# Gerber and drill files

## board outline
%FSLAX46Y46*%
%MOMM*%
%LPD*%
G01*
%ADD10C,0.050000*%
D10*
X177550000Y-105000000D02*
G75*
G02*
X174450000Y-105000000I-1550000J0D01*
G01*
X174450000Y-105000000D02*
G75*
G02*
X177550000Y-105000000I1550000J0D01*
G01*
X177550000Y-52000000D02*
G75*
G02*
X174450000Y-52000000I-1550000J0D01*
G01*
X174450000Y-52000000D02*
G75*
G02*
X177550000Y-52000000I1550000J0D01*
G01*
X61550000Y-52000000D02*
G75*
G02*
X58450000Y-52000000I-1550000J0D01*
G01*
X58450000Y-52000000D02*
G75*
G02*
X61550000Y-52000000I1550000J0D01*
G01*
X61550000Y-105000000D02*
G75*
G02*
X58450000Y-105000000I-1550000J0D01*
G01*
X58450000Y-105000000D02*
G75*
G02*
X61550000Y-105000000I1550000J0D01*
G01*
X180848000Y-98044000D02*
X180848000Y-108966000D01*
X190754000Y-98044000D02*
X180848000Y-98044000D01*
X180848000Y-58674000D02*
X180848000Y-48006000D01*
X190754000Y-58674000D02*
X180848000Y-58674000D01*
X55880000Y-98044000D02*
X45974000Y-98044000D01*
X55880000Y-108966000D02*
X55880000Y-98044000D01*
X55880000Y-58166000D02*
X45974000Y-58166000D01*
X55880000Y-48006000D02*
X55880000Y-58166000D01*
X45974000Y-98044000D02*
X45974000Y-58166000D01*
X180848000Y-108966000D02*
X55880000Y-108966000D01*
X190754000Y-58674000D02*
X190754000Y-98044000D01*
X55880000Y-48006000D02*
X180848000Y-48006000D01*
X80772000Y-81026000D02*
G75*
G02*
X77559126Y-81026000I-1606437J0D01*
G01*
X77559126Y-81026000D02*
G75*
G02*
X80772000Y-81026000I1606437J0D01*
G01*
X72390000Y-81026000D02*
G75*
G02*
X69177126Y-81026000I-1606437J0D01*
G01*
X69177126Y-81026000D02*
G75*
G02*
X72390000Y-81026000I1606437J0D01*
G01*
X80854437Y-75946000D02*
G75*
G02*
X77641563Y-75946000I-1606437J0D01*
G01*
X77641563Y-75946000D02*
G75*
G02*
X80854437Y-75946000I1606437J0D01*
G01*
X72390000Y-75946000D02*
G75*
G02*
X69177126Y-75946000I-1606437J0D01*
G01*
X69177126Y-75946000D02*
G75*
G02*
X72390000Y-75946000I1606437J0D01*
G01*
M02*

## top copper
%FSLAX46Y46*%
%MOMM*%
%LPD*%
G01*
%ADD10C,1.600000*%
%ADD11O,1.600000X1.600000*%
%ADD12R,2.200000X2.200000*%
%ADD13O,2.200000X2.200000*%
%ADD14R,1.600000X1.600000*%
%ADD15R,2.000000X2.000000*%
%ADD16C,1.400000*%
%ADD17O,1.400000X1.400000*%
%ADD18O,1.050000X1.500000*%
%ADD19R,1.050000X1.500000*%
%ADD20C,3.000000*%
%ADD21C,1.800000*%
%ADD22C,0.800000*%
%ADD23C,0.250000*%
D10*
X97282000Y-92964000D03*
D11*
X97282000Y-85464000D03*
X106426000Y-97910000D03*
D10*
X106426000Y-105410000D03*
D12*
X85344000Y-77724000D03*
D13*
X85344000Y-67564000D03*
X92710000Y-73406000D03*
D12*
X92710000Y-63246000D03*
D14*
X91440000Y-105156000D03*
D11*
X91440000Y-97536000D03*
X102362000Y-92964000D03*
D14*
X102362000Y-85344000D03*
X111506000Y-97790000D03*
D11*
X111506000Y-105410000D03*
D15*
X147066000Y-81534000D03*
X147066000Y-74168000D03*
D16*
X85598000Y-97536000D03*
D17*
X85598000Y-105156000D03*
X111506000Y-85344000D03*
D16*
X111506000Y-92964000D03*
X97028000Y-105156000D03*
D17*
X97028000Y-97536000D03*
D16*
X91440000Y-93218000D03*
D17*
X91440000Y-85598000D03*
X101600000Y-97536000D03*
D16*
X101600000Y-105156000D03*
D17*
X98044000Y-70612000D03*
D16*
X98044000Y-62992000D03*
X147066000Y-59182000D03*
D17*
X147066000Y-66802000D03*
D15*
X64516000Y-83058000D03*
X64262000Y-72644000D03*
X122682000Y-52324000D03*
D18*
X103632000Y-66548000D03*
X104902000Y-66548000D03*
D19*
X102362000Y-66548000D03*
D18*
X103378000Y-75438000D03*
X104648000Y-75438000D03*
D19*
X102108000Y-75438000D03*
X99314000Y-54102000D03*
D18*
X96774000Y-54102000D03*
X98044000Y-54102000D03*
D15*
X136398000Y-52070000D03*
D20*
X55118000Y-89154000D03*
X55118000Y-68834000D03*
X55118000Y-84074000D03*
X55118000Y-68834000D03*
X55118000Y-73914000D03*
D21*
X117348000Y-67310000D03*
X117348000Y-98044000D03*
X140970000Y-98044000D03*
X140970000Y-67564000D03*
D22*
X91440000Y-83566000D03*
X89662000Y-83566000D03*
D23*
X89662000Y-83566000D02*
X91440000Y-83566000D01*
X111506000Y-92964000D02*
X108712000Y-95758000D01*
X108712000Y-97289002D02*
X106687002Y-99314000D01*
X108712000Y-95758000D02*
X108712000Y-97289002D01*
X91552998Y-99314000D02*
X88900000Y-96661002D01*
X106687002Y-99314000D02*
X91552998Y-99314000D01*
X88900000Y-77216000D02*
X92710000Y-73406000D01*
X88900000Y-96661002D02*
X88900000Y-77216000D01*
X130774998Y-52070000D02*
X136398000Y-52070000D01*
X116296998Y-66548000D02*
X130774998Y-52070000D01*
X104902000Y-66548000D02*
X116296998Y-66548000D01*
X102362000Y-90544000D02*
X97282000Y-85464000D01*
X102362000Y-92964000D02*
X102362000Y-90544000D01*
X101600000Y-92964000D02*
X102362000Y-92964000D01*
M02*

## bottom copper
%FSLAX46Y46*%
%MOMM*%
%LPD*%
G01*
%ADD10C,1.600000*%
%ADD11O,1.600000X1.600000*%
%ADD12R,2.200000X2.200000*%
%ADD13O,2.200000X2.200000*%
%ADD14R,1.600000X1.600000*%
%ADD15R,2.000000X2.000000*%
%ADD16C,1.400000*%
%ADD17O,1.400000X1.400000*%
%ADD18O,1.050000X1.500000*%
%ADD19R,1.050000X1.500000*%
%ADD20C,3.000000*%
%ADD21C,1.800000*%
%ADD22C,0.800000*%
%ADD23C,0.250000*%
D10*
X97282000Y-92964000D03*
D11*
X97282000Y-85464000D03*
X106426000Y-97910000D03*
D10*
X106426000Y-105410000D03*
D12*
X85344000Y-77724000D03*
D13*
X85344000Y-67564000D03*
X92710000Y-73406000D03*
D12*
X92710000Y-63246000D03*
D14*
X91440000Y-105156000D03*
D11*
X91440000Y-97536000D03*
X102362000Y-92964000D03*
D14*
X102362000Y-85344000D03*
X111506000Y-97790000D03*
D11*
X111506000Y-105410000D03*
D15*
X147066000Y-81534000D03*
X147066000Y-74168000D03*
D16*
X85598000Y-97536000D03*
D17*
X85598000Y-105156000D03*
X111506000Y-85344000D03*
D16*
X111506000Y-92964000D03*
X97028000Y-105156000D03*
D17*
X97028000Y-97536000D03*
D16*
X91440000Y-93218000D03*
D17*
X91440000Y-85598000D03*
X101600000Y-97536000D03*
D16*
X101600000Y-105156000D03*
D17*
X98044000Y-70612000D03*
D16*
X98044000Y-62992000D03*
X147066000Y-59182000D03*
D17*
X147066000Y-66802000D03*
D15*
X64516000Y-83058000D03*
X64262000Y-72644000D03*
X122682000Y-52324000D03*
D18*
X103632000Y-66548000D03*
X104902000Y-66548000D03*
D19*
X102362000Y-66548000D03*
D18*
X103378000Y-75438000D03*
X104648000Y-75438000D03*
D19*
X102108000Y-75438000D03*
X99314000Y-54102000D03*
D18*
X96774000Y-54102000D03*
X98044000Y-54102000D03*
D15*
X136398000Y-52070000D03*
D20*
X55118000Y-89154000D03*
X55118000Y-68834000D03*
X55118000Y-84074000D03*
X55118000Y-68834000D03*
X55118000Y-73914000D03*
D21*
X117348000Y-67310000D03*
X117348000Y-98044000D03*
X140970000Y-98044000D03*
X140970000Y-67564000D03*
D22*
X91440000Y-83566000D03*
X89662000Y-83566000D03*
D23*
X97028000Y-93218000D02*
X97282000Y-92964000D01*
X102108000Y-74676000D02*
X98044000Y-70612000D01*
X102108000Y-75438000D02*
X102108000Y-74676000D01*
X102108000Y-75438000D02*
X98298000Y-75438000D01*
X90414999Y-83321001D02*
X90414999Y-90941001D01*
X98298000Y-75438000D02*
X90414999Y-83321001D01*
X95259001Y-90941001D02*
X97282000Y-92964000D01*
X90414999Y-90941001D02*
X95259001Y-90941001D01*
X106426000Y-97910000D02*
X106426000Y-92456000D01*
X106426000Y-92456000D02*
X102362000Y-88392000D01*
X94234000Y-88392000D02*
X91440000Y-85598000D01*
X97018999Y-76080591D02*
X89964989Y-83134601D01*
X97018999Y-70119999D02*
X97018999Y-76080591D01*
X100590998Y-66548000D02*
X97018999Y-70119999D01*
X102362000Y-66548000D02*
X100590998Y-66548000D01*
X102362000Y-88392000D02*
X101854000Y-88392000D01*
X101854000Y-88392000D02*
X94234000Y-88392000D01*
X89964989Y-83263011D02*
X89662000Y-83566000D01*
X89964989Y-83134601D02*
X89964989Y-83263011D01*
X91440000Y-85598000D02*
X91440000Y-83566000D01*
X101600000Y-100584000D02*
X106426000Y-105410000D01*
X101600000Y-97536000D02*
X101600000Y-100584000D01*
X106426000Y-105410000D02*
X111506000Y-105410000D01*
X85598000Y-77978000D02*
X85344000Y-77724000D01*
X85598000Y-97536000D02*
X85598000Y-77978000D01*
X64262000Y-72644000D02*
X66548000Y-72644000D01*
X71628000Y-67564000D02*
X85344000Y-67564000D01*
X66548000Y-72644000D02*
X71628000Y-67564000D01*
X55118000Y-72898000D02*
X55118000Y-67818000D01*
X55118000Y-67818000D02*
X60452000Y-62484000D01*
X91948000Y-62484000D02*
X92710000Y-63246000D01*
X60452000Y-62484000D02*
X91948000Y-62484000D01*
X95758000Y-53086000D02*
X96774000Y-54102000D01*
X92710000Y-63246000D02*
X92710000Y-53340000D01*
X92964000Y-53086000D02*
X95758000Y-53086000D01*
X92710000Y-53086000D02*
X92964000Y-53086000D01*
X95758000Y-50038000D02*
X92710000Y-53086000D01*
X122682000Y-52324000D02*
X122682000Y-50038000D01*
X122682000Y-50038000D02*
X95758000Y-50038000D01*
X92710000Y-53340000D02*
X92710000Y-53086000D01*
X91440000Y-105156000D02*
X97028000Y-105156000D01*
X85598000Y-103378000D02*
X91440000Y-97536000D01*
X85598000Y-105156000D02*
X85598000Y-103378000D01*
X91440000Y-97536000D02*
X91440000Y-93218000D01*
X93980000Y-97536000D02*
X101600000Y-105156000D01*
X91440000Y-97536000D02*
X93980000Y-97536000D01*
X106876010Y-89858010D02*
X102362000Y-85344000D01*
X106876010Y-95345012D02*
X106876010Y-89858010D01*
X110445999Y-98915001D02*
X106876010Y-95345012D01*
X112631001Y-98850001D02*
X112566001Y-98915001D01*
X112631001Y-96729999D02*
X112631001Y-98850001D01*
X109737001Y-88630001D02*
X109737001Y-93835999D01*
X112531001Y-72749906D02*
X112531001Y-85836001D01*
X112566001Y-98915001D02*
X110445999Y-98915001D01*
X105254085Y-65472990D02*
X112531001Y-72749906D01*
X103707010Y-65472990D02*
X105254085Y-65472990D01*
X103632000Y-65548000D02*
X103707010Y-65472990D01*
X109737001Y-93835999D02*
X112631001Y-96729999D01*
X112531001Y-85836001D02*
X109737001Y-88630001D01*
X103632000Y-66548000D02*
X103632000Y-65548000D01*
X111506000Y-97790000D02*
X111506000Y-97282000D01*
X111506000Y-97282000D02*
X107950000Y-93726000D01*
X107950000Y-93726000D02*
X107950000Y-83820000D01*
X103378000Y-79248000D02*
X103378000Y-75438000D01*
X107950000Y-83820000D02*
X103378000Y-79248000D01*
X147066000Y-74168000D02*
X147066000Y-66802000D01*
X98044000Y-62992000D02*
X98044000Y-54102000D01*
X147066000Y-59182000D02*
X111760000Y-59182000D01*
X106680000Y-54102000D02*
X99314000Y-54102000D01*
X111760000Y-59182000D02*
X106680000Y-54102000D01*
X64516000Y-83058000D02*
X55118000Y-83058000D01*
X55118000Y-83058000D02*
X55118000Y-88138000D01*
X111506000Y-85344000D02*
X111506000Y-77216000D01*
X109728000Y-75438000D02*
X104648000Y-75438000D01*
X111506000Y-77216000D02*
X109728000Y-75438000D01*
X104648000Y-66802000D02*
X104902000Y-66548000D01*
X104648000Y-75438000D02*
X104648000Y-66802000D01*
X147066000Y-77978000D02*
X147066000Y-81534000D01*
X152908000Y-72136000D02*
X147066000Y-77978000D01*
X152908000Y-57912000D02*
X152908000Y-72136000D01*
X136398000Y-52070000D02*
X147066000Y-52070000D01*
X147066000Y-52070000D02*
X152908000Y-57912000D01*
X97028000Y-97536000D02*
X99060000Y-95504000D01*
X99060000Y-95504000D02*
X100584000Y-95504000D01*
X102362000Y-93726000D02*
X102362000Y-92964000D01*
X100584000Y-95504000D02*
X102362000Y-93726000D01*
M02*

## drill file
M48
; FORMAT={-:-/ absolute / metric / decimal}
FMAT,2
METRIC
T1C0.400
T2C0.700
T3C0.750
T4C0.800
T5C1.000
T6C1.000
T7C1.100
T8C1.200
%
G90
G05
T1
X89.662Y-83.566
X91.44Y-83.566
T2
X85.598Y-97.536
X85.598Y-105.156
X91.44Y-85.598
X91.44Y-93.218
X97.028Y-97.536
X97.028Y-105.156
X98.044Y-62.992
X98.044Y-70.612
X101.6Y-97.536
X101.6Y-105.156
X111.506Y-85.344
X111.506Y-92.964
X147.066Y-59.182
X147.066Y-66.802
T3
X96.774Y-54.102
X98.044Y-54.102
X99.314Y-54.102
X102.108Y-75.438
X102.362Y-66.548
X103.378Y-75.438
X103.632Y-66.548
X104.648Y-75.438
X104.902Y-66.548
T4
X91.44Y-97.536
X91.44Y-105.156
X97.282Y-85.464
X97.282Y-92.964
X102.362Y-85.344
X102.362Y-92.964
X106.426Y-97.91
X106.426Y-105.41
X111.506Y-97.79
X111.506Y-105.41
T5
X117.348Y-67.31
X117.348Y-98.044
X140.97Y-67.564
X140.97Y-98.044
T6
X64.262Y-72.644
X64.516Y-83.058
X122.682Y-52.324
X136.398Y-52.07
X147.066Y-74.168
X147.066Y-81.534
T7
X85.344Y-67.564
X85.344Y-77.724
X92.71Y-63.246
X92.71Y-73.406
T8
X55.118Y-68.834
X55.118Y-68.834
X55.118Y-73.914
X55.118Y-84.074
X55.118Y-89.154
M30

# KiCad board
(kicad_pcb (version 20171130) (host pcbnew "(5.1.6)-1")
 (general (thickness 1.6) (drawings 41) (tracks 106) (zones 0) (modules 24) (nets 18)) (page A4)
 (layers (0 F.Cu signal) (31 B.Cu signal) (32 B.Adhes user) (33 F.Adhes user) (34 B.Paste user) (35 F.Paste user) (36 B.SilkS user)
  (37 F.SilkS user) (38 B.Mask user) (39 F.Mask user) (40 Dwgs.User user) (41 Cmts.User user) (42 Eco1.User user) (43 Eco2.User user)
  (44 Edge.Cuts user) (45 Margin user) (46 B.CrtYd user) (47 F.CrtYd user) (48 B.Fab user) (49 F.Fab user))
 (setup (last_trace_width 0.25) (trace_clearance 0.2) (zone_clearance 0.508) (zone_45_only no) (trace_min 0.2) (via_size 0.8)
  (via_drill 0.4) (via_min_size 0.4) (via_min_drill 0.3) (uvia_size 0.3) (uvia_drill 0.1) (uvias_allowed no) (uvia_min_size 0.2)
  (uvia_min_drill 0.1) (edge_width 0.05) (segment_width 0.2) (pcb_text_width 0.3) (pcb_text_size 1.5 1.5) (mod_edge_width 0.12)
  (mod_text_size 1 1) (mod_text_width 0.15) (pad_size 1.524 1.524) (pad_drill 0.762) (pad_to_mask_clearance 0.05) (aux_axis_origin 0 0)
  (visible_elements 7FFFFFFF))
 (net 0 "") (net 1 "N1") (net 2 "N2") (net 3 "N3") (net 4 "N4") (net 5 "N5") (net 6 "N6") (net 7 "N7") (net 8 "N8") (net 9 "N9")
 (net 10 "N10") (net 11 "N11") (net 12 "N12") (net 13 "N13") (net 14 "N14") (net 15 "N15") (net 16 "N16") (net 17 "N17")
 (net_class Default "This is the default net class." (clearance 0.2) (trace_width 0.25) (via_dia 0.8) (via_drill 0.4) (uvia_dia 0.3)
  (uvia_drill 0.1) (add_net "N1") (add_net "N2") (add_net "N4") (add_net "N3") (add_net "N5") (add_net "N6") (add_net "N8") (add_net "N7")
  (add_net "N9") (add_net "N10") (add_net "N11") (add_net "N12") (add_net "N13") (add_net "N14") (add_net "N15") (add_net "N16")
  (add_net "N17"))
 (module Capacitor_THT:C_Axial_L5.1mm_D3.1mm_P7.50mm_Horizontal (layer F.Cu) (at 97.282 92.964 90)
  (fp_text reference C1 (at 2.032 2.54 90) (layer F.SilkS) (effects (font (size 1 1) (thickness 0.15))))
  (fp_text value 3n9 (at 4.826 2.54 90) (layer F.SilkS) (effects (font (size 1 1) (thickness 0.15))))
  (pad 1 thru_hole circle (at 0 0 90) (size 1.6 1.6) (drill 0.8) (layers *.Cu *.Mask) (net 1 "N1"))
  (pad 2 thru_hole oval (at 7.5 0 90) (size 1.6 1.6) (drill 0.8) (layers *.Cu *.Mask) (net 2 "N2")))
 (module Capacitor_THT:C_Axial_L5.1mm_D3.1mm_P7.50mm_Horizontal (layer F.Cu) (at 106.426 105.41 90)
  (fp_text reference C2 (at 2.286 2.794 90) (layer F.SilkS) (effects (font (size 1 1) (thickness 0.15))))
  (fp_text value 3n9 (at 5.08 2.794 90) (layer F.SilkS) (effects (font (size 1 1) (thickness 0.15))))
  (pad 2 thru_hole oval (at 7.5 0 90) (size 1.6 1.6) (drill 0.8) (layers *.Cu *.Mask) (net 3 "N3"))
  (pad 1 thru_hole circle (at 0 0 90) (size 1.6 1.6) (drill 0.8) (layers *.Cu *.Mask) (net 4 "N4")))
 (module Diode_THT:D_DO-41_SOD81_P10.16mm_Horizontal (layer F.Cu) (at 85.344 77.724 90)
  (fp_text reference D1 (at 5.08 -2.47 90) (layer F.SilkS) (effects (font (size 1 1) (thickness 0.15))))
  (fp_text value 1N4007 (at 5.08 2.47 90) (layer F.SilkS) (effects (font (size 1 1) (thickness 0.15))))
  (pad 1 thru_hole rect (at 0 0 90) (size 2.2 2.2) (drill 1.1) (layers *.Cu *.Mask) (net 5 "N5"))
  (pad 2 thru_hole oval (at 10.16 0 90) (size 2.2 2.2) (drill 1.1) (layers *.Cu *.Mask) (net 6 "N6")))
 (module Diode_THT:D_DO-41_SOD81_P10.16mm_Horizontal (layer F.Cu) (at 92.71 63.246 270)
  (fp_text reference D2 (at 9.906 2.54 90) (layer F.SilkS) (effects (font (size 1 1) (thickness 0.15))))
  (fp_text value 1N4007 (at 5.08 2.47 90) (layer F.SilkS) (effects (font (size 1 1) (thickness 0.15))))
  (pad 2 thru_hole oval (at 10.16 0 270) (size 2.2 2.2) (drill 1.1) (layers *.Cu *.Mask) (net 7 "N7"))
  (pad 1 thru_hole rect (at 0 0 270) (size 2.2 2.2) (drill 1.1) (layers *.Cu *.Mask) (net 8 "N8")))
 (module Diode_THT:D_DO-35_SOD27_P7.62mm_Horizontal (layer F.Cu) (at 91.44 105.156 90)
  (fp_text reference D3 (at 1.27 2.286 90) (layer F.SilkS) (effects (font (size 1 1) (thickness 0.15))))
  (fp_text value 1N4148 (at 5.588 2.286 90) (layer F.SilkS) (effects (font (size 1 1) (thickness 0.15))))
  (pad 1 thru_hole rect (at 0 0 90) (size 1.6 1.6) (drill 0.8) (layers *.Cu *.Mask) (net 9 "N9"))
  (pad 2 thru_hole oval (at 7.62 0 90) (size 1.6 1.6) (drill 0.8) (layers *.Cu *.Mask) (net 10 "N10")))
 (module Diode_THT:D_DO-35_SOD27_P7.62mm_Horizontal (layer F.Cu) (at 102.362 85.344 270)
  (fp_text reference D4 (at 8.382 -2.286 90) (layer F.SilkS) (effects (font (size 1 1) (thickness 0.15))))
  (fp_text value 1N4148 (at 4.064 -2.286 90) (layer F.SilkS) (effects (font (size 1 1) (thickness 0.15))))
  (pad 2 thru_hole oval (at 7.62 0 270) (size 1.6 1.6) (drill 0.8) (layers *.Cu *.Mask) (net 2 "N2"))
  (pad 1 thru_hole rect (at 0 0 270) (size 1.6 1.6) (drill 0.8) (layers *.Cu *.Mask) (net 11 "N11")))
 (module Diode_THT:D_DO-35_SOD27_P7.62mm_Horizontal (layer F.Cu) (at 111.506 97.79 270)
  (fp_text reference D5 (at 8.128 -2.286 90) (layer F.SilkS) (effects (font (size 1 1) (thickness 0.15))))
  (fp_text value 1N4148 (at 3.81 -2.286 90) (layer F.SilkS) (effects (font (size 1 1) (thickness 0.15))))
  (pad 1 thru_hole rect (at 0 0 270) (size 1.6 1.6) (drill 0.8) (layers *.Cu *.Mask) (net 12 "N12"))
  (pad 2 thru_hole oval (at 7.62 0 270) (size 1.6 1.6) (drill 0.8) (layers *.Cu *.Mask) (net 4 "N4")))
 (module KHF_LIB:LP (layer F.Cu) (at 147.066 81.534)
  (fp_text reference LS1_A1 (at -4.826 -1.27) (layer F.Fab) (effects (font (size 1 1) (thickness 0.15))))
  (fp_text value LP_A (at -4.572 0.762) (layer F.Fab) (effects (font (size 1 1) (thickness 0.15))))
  (pad 1 thru_hole rect (at 0 0) (size 2 2) (drill 1) (layers *.Cu *.Mask) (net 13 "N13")))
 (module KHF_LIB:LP (layer F.Cu) (at 147.066 74.168)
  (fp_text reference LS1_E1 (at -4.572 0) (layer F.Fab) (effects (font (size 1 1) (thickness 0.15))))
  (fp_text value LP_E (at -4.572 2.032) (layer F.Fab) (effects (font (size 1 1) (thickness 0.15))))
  (pad 1 thru_hole rect (at 0 0) (size 2 2) (drill 1) (layers *.Cu *.Mask) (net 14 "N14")))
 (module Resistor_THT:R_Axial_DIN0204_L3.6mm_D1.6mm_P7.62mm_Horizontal (layer F.Cu) (at 85.598 97.536 270)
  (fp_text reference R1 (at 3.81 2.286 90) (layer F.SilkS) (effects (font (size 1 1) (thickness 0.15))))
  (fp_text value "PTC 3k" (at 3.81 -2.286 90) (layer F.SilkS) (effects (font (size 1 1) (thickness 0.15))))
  (pad 1 thru_hole circle (at 0 0 270) (size 1.4 1.4) (drill 0.7) (layers *.Cu *.Mask) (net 5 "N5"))
  (pad 2 thru_hole oval (at 7.62 0 270) (size 1.4 1.4) (drill 0.7) (layers *.Cu *.Mask) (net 10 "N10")))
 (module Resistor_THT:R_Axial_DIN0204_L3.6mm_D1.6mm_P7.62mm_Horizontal (layer F.Cu) (at 111.506 92.964 90)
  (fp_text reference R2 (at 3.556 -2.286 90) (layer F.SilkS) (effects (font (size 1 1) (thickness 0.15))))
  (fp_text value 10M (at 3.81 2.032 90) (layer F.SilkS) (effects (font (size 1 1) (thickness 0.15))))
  (pad 2 thru_hole oval (at 7.62 0 90) (size 1.4 1.4) (drill 0.7) (layers *.Cu *.Mask) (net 13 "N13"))
  (pad 1 thru_hole circle (at 0 0 90) (size 1.4 1.4) (drill 0.7) (layers *.Cu *.Mask) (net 7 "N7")))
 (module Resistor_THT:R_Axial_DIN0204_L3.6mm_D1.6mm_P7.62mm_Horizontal (layer F.Cu) (at 97.028 105.156 90)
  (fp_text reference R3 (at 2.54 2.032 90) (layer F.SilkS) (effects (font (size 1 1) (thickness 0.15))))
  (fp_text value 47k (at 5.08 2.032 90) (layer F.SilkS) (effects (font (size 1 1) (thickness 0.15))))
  (pad 1 thru_hole circle (at 0 0 90) (size 1.4 1.4) (drill 0.7) (layers *.Cu *.Mask) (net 9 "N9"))
  (pad 2 thru_hole oval (at 7.62 0 90) (size 1.4 1.4) (drill 0.7) (layers *.Cu *.Mask) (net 2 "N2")))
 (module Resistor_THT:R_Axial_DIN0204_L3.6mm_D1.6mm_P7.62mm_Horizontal (layer F.Cu) (at 91.44 93.218 90)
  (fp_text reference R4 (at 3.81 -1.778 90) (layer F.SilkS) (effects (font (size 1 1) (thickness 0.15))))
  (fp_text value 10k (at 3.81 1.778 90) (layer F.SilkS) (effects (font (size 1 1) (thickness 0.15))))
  (pad 1 thru_hole circle (at 0 0 90) (size 1.4 1.4) (drill 0.7) (layers *.Cu *.Mask) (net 10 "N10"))
  (pad 2 thru_hole oval (at 7.62 0 90) (size 1.4 1.4) (drill 0.7) (layers *.Cu *.Mask) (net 3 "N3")))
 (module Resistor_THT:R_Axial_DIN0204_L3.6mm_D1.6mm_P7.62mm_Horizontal (layer F.Cu) (at 101.6 105.156 90)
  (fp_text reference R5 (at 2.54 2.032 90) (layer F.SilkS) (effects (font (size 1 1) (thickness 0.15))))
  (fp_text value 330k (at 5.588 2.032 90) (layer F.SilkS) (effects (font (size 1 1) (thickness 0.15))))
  (pad 2 thru_hole oval (at 7.62 0 90) (size 1.4 1.4) (drill 0.7) (layers *.Cu *.Mask) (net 4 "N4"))
  (pad 1 thru_hole circle (at 0 0 90) (size 1.4 1.4) (drill 0.7) (layers *.Cu *.Mask) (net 10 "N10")))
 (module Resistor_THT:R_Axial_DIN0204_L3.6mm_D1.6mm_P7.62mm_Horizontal (layer F.Cu) (at 98.044 62.992 270)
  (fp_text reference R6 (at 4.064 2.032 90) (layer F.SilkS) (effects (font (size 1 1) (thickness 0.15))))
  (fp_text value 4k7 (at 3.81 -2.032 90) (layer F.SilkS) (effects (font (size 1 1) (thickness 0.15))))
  (pad 2 thru_hole oval (at 7.62 0 270) (size 1.4 1.4) (drill 0.7) (layers *.Cu *.Mask) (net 1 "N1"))
  (pad 1 thru_hole circle (at 0 0 270) (size 1.4 1.4) (drill 0.7) (layers *.Cu *.Mask) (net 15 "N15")))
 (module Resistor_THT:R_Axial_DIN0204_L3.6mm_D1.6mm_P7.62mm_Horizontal (layer F.Cu) (at 147.066 59.182 270)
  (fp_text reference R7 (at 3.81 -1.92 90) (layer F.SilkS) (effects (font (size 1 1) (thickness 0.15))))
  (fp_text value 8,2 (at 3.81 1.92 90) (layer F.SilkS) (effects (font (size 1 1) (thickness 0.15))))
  (pad 1 thru_hole circle (at 0 0 270) (size 1.4 1.4) (drill 0.7) (layers *.Cu *.Mask) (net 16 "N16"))
  (pad 2 thru_hole oval (at 7.62 0 270) (size 1.4 1.4) (drill 0.7) (layers *.Cu *.Mask) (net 14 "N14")))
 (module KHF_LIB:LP (layer F.Cu) (at 64.516 83.058)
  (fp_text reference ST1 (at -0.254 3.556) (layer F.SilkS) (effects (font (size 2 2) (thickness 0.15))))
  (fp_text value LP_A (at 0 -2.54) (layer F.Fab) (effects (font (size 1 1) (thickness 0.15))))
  (pad 1 thru_hole rect (at 0 0) (size 2 2) (drill 1) (layers *.Cu *.Mask) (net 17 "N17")))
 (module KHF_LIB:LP (layer F.Cu) (at 64.262 72.644)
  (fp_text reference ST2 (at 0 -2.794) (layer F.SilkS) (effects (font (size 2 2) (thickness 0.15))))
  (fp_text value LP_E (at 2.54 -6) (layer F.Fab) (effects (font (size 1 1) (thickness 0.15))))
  (pad 1 thru_hole rect (at 0 0) (size 2 2) (drill 1) (layers *.Cu *.Mask) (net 6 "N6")))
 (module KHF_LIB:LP (layer F.Cu) (at 122.682 52.324)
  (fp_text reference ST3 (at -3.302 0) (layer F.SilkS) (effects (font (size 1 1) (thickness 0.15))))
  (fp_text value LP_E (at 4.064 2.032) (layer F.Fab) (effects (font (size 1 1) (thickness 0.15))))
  (pad 1 thru_hole rect (at 0 0) (size 2 2) (drill 1) (layers *.Cu *.Mask) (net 8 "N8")))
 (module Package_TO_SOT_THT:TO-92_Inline (layer F.Cu) (at 102.362 66.548)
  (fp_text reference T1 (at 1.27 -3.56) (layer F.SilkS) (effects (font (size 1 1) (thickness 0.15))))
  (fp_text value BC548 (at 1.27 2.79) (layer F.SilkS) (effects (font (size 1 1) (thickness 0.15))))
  (pad 2 thru_hole oval (at 1.27 0) (size 1.05 1.5) (drill 0.75) (layers *.Cu *.Mask) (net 11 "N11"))
  (pad 3 thru_hole oval (at 2.54 0) (size 1.05 1.5) (drill 0.75) (layers *.Cu *.Mask) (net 13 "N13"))
  (pad 1 thru_hole rect (at 0 0) (size 1.05 1.5) (drill 0.75) (layers *.Cu *.Mask) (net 3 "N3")))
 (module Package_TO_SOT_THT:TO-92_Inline (layer F.Cu) (at 102.108 75.438)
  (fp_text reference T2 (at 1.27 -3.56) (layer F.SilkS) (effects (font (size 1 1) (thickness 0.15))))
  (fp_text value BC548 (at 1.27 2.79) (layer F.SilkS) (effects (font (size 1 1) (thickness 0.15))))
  (pad 2 thru_hole oval (at 1.27 0) (size 1.05 1.5) (drill 0.75) (layers *.Cu *.Mask) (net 12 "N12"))
  (pad 3 thru_hole oval (at 2.54 0) (size 1.05 1.5) (drill 0.75) (layers *.Cu *.Mask) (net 13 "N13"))
  (pad 1 thru_hole rect (at 0 0) (size 1.05 1.5) (drill 0.75) (layers *.Cu *.Mask) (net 1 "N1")))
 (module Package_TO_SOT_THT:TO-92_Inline (layer F.Cu) (at 99.314 54.102 180)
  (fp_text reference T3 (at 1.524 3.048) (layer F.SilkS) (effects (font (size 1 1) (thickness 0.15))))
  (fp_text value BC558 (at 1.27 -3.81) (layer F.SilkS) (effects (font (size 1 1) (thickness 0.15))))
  (pad 1 thru_hole rect (at 0 0 180) (size 1.05 1.5) (drill 0.75) (layers *.Cu *.Mask) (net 16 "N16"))
  (pad 3 thru_hole oval (at 2.54 0 180) (size 1.05 1.5) (drill 0.75) (layers *.Cu *.Mask) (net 8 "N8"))
  (pad 2 thru_hole oval (at 1.27 0 180) (size 1.05 1.5) (drill 0.75) (layers *.Cu *.Mask) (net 15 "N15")))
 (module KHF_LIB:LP (layer F.Cu) (at 136.398 52.07)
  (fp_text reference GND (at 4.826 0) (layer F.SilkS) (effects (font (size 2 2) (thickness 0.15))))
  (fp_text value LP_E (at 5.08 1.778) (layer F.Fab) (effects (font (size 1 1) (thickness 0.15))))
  (pad 1 thru_hole rect (at 0 0) (size 2 2) (drill 1) (layers *.Cu *.Mask) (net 13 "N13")))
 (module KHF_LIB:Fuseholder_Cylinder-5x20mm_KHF (layer F.Cu) (at 55.118 89.154 90)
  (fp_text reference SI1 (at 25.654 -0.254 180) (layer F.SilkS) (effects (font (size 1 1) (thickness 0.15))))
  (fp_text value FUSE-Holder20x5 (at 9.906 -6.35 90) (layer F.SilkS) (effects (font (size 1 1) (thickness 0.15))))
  (pad 1 thru_hole circle (at 0 0 90) (size 3 3) (drill 1.2) (layers *.Cu *.Mask) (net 17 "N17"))
  (pad 2 thru_hole circle (at 20.32 0 90) (size 3 3) (drill 1.2) (layers *.Cu *.Mask) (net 8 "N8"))
  (pad 1 thru_hole circle (at 5.08 0 90) (size 3 3) (drill 1.2) (layers *.Cu *.Mask) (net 17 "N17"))
  (pad 2 thru_hole circle (at 20.32 0 90) (size 3 3) (drill 1.2) (layers *.Cu *.Mask) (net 8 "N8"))
  (pad 2 thru_hole circle (at 15.24 0 90) (size 3 3) (drill 1.2) (layers *.Cu *.Mask) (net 8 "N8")))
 (gr_circle (center 176 105) (end 177.55 105) (layer Edge.Cuts) (width 0.05))
 (gr_circle (center 176 52) (end 177.55 52) (layer Edge.Cuts) (width 0.05))
 (gr_circle (center 60 52) (end 61.55 52) (layer Edge.Cuts) (width 0.05))
 (gr_circle (center 60 105) (end 61.55 105) (layer Edge.Cuts) (width 0.05))
 (gr_line (start 180.848 98.044) (end 180.848 108.966) (layer Edge.Cuts) (width 0.05))
 (gr_line (start 190.754 98.044) (end 180.848 98.044) (layer Edge.Cuts) (width 0.05))
 (gr_line (start 180.848 58.674) (end 180.848 48.006) (layer Edge.Cuts) (width 0.05))
 (gr_line (start 190.754 58.674) (end 180.848 58.674) (layer Edge.Cuts) (width 0.05))
 (gr_line (start 55.88 98.044) (end 45.974 98.044) (layer Edge.Cuts) (width 0.05))
 (gr_line (start 55.88 108.966) (end 55.88 98.044) (layer Edge.Cuts) (width 0.05))
 (gr_line (start 55.88 58.166) (end 45.974 58.166) (layer Edge.Cuts) (width 0.05))
 (gr_line (start 55.88 48.006) (end 55.88 58.166) (layer Edge.Cuts) (width 0.05))
 (gr_line (start 45.974 98.044) (end 45.974 58.166) (layer Edge.Cuts) (width 0.05))
 (gr_line (start 180.848 108.966) (end 55.88 108.966) (layer Edge.Cuts) (width 0.05))
 (gr_line (start 190.754 58.674) (end 190.754 98.044) (layer Edge.Cuts) (width 0.05))
 (gr_line (start 55.88 48.006) (end 180.848 48.006) (layer Edge.Cuts) (width 0.05))
 (gr_circle (center 79.165563 81.026) (end 77.641563 80.518) (layer Edge.Cuts) (width 0.05))
 (gr_circle (center 70.783563 81.026) (end 69.259563 80.518) (layer Edge.Cuts) (width 0.05))
 (gr_circle (center 79.248 75.946) (end 77.724 75.438) (layer Edge.Cuts) (width 0.05))
 (gr_circle (center 70.783563 75.946) (end 69.259563 75.438) (layer Edge.Cuts) (width 0.05))
 (via (at 117.348 67.31) (size 1.8) (drill 1) (layers F.Cu B.Cu) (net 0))
 (via (at 117.348 98.044) (size 1.8) (drill 1) (layers F.Cu B.Cu) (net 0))
 (via (at 140.97 98.044) (size 1.8) (drill 1) (layers F.Cu B.Cu) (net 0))
 (via (at 140.97 67.564) (size 1.8) (drill 1) (layers F.Cu B.Cu) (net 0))
 (segment (start 97.028 93.218) (end 97.282 92.964) (width 0.25) (layer B.Cu) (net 1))
 (segment (start 102.108 74.676) (end 98.044 70.612) (width 0.25) (layer B.Cu) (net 1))
 (segment (start 102.108 75.438) (end 102.108 74.676) (width 0.25) (layer B.Cu) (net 1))
 (segment (start 102.108 75.438) (end 98.298 75.438) (width 0.25) (layer B.Cu) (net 1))
 (segment (start 90.414999 83.321001) (end 90.414999 90.941001) (width 0.25) (layer B.Cu) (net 1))
 (segment (start 98.298 75.438) (end 90.414999 83.321001) (width 0.25) (layer B.Cu) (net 1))
 (segment (start 95.259001 90.941001) (end 97.282 92.964) (width 0.25) (layer B.Cu) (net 1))
 (segment (start 90.414999 90.941001) (end 95.259001 90.941001) (width 0.25) (layer B.Cu) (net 1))
 (via (at 91.44 83.566) (size 0.8) (drill 0.4) (layers F.Cu B.Cu) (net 3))
 (via (at 89.662 83.566) (size 0.8) (drill 0.4) (layers F.Cu B.Cu) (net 3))
 (segment (start 106.426 97.91) (end 106.426 92.456) (width 0.25) (layer B.Cu) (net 3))
 (segment (start 106.426 92.456) (end 102.362 88.392) (width 0.25) (layer B.Cu) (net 3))
 (segment (start 94.234 88.392) (end 91.44 85.598) (width 0.25) (layer B.Cu) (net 3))
 (segment (start 97.018999 76.080591) (end 89.964989 83.134601) (width 0.25) (layer B.Cu) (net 3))
 (segment (start 97.018999 70.119999) (end 97.018999 76.080591) (width 0.25) (layer B.Cu) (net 3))
 (segment (start 100.590998 66.548) (end 97.018999 70.119999) (width 0.25) (layer B.Cu) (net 3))
 (segment (start 102.362 66.548) (end 100.590998 66.548) (width 0.25) (layer B.Cu) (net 3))
 (segment (start 102.362 88.392) (end 101.854 88.392) (width 0.25) (layer B.Cu) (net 3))
 (segment (start 101.854 88.392) (end 94.234 88.392) (width 0.25) (layer B.Cu) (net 3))
 (segment (start 89.964989 83.263011) (end 89.662 83.566) (width 0.25) (layer B.Cu) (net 3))
 (segment (start 89.964989 83.134601) (end 89.964989 83.263011) (width 0.25) (layer B.Cu) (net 3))
 (segment (start 91.44 85.598) (end 91.44 83.566) (width 0.25) (layer B.Cu) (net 3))
 (segment (start 89.662 83.566) (end 91.44 83.566) (width 0.25) (layer F.Cu) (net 3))
 (segment (start 101.6 100.584) (end 106.426 105.41) (width 0.25) (layer B.Cu) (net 4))
 (segment (start 101.6 97.536) (end 101.6 100.584) (width 0.25) (layer B.Cu) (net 4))
 (segment (start 106.426 105.41) (end 111.506 105.41) (width 0.25) (layer B.Cu) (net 4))
 (segment (start 85.598 77.978) (end 85.344 77.724) (width 0.25) (layer B.Cu) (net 5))
 (segment (start 85.598 97.536) (end 85.598 77.978) (width 0.25) (layer B.Cu) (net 5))
 (segment (start 64.262 72.644) (end 66.548 72.644) (width 0.25) (layer B.Cu) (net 6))
 (segment (start 71.628 67.564) (end 85.344 67.564) (width 0.25) (layer B.Cu) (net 6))
 (segment (start 66.548 72.644) (end 71.628 67.564) (width 0.25) (layer B.Cu) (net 6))
 (segment (start 111.506 92.964) (end 108.712 95.758) (width 0.25) (layer F.Cu) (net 7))
 (segment (start 108.712 97.289002) (end 106.687002 99.314) (width 0.25) (layer F.Cu) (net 7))
 (segment (start 108.712 95.758) (end 108.712 97.289002) (width 0.25) (layer F.Cu) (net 7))
 (segment (start 91.552998 99.314) (end 88.9 96.661002) (width 0.25) (layer F.Cu) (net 7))
 (segment (start 106.687002 99.314) (end 91.552998 99.314) (width 0.25) (layer F.Cu) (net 7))
 (segment (start 88.9 77.216) (end 92.71 73.406) (width 0.25) (layer F.Cu) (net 7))
 (segment (start 88.9 96.661002) (end 88.9 77.216) (width 0.25) (layer F.Cu) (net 7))
 (segment (start 55.118 72.898) (end 55.118 67.818) (width 0.25) (layer B.Cu) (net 8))
 (segment (start 55.118 67.818) (end 60.452 62.484) (width 0.25) (layer B.Cu) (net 8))
 (segment (start 91.948 62.484) (end 92.71 63.246) (width 0.25) (layer B.Cu) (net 8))
 (segment (start 60.452 62.484) (end 91.948 62.484) (width 0.25) (layer B.Cu) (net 8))
 (segment (start 95.758 53.086) (end 96.774 54.102) (width 0.25) (layer B.Cu) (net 8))
 (segment (start 92.71 63.246) (end 92.71 53.34) (width 0.25) (layer B.Cu) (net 8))
 (segment (start 92.964 53.086) (end 95.758 53.086) (width 0.25) (layer B.Cu) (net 8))
 (segment (start 92.71 53.086) (end 92.964 53.086) (width 0.25) (layer B.Cu) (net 8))
 (segment (start 95.758 50.038) (end 92.71 53.086) (width 0.25) (layer B.Cu) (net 8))
 (segment (start 122.682 52.324) (end 122.682 50.038) (width 0.25) (layer B.Cu) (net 8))
 (segment (start 122.682 50.038) (end 95.758 50.038) (width 0.25) (layer B.Cu) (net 8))
 (segment (start 92.71 53.34) (end 92.71 53.086) (width 0.25) (layer B.Cu) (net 8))
 (segment (start 91.44 105.156) (end 97.028 105.156) (width 0.25) (layer B.Cu) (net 9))
 (segment (start 85.598 103.378) (end 91.44 97.536) (width 0.25) (layer B.Cu) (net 10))
 (segment (start 85.598 105.156) (end 85.598 103.378) (width 0.25) (layer B.Cu) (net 10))
 (segment (start 91.44 97.536) (end 91.44 93.218) (width 0.25) (layer B.Cu) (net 10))
 (segment (start 93.98 97.536) (end 101.6 105.156) (width 0.25) (layer B.Cu) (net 10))
 (segment (start 91.44 97.536) (end 93.98 97.536) (width 0.25) (layer B.Cu) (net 10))
 (segment (start 106.87601 89.85801) (end 102.362 85.344) (width 0.25) (layer B.Cu) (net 11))
 (segment (start 106.87601 95.345012) (end 106.87601 89.85801) (width 0.25) (layer B.Cu) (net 11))
 (segment (start 110.445999 98.915001) (end 106.87601 95.345012) (width 0.25) (layer B.Cu) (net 11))
 (segment (start 112.631001 98.850001) (end 112.566001 98.915001) (width 0.25) (layer B.Cu) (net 11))
 (segment (start 112.631001 96.729999) (end 112.631001 98.850001) (width 0.25) (layer B.Cu) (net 11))
 (segment (start 109.737001 88.630001) (end 109.737001 93.835999) (width 0.25) (layer B.Cu) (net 11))
 (segment (start 112.531001 72.749906) (end 112.531001 85.836001) (width 0.25) (layer B.Cu) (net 11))
 (segment (start 112.566001 98.915001) (end 110.445999 98.915001) (width 0.25) (layer B.Cu) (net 11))
 (segment (start 105.254085 65.47299) (end 112.531001 72.749906) (width 0.25) (layer B.Cu) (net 11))
 (segment (start 103.70701 65.47299) (end 105.254085 65.47299) (width 0.25) (layer B.Cu) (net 11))
 (segment (start 103.632 65.548) (end 103.70701 65.47299) (width 0.25) (layer B.Cu) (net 11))
 (segment (start 109.737001 93.835999) (end 112.631001 96.729999) (width 0.25) (layer B.Cu) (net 11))
 (segment (start 112.531001 85.836001) (end 109.737001 88.630001) (width 0.25) (layer B.Cu) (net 11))
 (segment (start 103.632 66.548) (end 103.632 65.548) (width 0.25) (layer B.Cu) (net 11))
 (segment (start 111.506 97.79) (end 111.506 97.282) (width 0.25) (layer B.Cu) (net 12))
 (segment (start 111.506 97.282) (end 107.95 93.726) (width 0.25) (layer B.Cu) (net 12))
 (segment (start 107.95 93.726) (end 107.95 83.82) (width 0.25) (layer B.Cu) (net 12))
 (segment (start 103.378 79.248) (end 103.378 75.438) (width 0.25) (layer B.Cu) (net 12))
 (segment (start 107.95 83.82) (end 103.378 79.248) (width 0.25) (layer B.Cu) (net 12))
 (segment (start 147.066 74.168) (end 147.066 66.802) (width 0.25) (layer B.Cu) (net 14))
 (segment (start 98.044 62.992) (end 98.044 54.102) (width 0.25) (layer B.Cu) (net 15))
 (segment (start 147.066 59.182) (end 111.76 59.182) (width 0.25) (layer B.Cu) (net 16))
 (segment (start 106.68 54.102) (end 99.314 54.102) (width 0.25) (layer B.Cu) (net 16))
 (segment (start 111.76 59.182) (end 106.68 54.102) (width 0.25) (layer B.Cu) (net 16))
 (segment (start 64.516 83.058) (end 55.118 83.058) (width 0.25) (layer B.Cu) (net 17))
 (segment (start 55.118 83.058) (end 55.118 88.138) (width 0.25) (layer B.Cu) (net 17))
 (segment (start 111.506 85.344) (end 111.506 77.216) (width 0.25) (layer B.Cu) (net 13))
 (segment (start 109.728 75.438) (end 104.648 75.438) (width 0.25) (layer B.Cu) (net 13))
 (segment (start 111.506 77.216) (end 109.728 75.438) (width 0.25) (layer B.Cu) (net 13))
 (segment (start 104.648 66.802) (end 104.902 66.548) (width 0.25) (layer B.Cu) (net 13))
 (segment (start 104.648 75.438) (end 104.648 66.802) (width 0.25) (layer B.Cu) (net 13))
 (segment (start 130.774998 52.07) (end 136.398 52.07) (width 0.25) (layer F.Cu) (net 13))
 (segment (start 116.296998 66.548) (end 130.774998 52.07) (width 0.25) (layer F.Cu) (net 13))
 (segment (start 104.902 66.548) (end 116.296998 66.548) (width 0.25) (layer F.Cu) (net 13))
 (segment (start 147.066 77.978) (end 147.066 81.534) (width 0.25) (layer B.Cu) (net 13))
 (segment (start 152.908 72.136) (end 147.066 77.978) (width 0.25) (layer B.Cu) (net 13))
 (segment (start 152.908 57.912) (end 152.908 72.136) (width 0.25) (layer B.Cu) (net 13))
 (segment (start 136.398 52.07) (end 147.066 52.07) (width 0.25) (layer B.Cu) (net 13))
 (segment (start 147.066 52.07) (end 152.908 57.912) (width 0.25) (layer B.Cu) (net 13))
 (segment (start 102.362 90.544) (end 97.282 85.464) (width 0.25) (layer F.Cu) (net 2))
 (segment (start 102.362 92.964) (end 102.362 90.544) (width 0.25) (layer F.Cu) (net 2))
 (segment (start 101.6 92.964) (end 102.362 92.964) (width 0.25) (layer F.Cu) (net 2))
 (segment (start 97.028 97.536) (end 99.06 95.504) (width 0.25) (layer B.Cu) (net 2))
 (segment (start 99.06 95.504) (end 100.584 95.504) (width 0.25) (layer B.Cu) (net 2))
 (segment (start 102.362 93.726) (end 102.362 92.964) (width 0.25) (layer B.Cu) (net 2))
 (segment (start 100.584 95.504) (end 102.362 93.726) (width 0.25) (layer B.Cu) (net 2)))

